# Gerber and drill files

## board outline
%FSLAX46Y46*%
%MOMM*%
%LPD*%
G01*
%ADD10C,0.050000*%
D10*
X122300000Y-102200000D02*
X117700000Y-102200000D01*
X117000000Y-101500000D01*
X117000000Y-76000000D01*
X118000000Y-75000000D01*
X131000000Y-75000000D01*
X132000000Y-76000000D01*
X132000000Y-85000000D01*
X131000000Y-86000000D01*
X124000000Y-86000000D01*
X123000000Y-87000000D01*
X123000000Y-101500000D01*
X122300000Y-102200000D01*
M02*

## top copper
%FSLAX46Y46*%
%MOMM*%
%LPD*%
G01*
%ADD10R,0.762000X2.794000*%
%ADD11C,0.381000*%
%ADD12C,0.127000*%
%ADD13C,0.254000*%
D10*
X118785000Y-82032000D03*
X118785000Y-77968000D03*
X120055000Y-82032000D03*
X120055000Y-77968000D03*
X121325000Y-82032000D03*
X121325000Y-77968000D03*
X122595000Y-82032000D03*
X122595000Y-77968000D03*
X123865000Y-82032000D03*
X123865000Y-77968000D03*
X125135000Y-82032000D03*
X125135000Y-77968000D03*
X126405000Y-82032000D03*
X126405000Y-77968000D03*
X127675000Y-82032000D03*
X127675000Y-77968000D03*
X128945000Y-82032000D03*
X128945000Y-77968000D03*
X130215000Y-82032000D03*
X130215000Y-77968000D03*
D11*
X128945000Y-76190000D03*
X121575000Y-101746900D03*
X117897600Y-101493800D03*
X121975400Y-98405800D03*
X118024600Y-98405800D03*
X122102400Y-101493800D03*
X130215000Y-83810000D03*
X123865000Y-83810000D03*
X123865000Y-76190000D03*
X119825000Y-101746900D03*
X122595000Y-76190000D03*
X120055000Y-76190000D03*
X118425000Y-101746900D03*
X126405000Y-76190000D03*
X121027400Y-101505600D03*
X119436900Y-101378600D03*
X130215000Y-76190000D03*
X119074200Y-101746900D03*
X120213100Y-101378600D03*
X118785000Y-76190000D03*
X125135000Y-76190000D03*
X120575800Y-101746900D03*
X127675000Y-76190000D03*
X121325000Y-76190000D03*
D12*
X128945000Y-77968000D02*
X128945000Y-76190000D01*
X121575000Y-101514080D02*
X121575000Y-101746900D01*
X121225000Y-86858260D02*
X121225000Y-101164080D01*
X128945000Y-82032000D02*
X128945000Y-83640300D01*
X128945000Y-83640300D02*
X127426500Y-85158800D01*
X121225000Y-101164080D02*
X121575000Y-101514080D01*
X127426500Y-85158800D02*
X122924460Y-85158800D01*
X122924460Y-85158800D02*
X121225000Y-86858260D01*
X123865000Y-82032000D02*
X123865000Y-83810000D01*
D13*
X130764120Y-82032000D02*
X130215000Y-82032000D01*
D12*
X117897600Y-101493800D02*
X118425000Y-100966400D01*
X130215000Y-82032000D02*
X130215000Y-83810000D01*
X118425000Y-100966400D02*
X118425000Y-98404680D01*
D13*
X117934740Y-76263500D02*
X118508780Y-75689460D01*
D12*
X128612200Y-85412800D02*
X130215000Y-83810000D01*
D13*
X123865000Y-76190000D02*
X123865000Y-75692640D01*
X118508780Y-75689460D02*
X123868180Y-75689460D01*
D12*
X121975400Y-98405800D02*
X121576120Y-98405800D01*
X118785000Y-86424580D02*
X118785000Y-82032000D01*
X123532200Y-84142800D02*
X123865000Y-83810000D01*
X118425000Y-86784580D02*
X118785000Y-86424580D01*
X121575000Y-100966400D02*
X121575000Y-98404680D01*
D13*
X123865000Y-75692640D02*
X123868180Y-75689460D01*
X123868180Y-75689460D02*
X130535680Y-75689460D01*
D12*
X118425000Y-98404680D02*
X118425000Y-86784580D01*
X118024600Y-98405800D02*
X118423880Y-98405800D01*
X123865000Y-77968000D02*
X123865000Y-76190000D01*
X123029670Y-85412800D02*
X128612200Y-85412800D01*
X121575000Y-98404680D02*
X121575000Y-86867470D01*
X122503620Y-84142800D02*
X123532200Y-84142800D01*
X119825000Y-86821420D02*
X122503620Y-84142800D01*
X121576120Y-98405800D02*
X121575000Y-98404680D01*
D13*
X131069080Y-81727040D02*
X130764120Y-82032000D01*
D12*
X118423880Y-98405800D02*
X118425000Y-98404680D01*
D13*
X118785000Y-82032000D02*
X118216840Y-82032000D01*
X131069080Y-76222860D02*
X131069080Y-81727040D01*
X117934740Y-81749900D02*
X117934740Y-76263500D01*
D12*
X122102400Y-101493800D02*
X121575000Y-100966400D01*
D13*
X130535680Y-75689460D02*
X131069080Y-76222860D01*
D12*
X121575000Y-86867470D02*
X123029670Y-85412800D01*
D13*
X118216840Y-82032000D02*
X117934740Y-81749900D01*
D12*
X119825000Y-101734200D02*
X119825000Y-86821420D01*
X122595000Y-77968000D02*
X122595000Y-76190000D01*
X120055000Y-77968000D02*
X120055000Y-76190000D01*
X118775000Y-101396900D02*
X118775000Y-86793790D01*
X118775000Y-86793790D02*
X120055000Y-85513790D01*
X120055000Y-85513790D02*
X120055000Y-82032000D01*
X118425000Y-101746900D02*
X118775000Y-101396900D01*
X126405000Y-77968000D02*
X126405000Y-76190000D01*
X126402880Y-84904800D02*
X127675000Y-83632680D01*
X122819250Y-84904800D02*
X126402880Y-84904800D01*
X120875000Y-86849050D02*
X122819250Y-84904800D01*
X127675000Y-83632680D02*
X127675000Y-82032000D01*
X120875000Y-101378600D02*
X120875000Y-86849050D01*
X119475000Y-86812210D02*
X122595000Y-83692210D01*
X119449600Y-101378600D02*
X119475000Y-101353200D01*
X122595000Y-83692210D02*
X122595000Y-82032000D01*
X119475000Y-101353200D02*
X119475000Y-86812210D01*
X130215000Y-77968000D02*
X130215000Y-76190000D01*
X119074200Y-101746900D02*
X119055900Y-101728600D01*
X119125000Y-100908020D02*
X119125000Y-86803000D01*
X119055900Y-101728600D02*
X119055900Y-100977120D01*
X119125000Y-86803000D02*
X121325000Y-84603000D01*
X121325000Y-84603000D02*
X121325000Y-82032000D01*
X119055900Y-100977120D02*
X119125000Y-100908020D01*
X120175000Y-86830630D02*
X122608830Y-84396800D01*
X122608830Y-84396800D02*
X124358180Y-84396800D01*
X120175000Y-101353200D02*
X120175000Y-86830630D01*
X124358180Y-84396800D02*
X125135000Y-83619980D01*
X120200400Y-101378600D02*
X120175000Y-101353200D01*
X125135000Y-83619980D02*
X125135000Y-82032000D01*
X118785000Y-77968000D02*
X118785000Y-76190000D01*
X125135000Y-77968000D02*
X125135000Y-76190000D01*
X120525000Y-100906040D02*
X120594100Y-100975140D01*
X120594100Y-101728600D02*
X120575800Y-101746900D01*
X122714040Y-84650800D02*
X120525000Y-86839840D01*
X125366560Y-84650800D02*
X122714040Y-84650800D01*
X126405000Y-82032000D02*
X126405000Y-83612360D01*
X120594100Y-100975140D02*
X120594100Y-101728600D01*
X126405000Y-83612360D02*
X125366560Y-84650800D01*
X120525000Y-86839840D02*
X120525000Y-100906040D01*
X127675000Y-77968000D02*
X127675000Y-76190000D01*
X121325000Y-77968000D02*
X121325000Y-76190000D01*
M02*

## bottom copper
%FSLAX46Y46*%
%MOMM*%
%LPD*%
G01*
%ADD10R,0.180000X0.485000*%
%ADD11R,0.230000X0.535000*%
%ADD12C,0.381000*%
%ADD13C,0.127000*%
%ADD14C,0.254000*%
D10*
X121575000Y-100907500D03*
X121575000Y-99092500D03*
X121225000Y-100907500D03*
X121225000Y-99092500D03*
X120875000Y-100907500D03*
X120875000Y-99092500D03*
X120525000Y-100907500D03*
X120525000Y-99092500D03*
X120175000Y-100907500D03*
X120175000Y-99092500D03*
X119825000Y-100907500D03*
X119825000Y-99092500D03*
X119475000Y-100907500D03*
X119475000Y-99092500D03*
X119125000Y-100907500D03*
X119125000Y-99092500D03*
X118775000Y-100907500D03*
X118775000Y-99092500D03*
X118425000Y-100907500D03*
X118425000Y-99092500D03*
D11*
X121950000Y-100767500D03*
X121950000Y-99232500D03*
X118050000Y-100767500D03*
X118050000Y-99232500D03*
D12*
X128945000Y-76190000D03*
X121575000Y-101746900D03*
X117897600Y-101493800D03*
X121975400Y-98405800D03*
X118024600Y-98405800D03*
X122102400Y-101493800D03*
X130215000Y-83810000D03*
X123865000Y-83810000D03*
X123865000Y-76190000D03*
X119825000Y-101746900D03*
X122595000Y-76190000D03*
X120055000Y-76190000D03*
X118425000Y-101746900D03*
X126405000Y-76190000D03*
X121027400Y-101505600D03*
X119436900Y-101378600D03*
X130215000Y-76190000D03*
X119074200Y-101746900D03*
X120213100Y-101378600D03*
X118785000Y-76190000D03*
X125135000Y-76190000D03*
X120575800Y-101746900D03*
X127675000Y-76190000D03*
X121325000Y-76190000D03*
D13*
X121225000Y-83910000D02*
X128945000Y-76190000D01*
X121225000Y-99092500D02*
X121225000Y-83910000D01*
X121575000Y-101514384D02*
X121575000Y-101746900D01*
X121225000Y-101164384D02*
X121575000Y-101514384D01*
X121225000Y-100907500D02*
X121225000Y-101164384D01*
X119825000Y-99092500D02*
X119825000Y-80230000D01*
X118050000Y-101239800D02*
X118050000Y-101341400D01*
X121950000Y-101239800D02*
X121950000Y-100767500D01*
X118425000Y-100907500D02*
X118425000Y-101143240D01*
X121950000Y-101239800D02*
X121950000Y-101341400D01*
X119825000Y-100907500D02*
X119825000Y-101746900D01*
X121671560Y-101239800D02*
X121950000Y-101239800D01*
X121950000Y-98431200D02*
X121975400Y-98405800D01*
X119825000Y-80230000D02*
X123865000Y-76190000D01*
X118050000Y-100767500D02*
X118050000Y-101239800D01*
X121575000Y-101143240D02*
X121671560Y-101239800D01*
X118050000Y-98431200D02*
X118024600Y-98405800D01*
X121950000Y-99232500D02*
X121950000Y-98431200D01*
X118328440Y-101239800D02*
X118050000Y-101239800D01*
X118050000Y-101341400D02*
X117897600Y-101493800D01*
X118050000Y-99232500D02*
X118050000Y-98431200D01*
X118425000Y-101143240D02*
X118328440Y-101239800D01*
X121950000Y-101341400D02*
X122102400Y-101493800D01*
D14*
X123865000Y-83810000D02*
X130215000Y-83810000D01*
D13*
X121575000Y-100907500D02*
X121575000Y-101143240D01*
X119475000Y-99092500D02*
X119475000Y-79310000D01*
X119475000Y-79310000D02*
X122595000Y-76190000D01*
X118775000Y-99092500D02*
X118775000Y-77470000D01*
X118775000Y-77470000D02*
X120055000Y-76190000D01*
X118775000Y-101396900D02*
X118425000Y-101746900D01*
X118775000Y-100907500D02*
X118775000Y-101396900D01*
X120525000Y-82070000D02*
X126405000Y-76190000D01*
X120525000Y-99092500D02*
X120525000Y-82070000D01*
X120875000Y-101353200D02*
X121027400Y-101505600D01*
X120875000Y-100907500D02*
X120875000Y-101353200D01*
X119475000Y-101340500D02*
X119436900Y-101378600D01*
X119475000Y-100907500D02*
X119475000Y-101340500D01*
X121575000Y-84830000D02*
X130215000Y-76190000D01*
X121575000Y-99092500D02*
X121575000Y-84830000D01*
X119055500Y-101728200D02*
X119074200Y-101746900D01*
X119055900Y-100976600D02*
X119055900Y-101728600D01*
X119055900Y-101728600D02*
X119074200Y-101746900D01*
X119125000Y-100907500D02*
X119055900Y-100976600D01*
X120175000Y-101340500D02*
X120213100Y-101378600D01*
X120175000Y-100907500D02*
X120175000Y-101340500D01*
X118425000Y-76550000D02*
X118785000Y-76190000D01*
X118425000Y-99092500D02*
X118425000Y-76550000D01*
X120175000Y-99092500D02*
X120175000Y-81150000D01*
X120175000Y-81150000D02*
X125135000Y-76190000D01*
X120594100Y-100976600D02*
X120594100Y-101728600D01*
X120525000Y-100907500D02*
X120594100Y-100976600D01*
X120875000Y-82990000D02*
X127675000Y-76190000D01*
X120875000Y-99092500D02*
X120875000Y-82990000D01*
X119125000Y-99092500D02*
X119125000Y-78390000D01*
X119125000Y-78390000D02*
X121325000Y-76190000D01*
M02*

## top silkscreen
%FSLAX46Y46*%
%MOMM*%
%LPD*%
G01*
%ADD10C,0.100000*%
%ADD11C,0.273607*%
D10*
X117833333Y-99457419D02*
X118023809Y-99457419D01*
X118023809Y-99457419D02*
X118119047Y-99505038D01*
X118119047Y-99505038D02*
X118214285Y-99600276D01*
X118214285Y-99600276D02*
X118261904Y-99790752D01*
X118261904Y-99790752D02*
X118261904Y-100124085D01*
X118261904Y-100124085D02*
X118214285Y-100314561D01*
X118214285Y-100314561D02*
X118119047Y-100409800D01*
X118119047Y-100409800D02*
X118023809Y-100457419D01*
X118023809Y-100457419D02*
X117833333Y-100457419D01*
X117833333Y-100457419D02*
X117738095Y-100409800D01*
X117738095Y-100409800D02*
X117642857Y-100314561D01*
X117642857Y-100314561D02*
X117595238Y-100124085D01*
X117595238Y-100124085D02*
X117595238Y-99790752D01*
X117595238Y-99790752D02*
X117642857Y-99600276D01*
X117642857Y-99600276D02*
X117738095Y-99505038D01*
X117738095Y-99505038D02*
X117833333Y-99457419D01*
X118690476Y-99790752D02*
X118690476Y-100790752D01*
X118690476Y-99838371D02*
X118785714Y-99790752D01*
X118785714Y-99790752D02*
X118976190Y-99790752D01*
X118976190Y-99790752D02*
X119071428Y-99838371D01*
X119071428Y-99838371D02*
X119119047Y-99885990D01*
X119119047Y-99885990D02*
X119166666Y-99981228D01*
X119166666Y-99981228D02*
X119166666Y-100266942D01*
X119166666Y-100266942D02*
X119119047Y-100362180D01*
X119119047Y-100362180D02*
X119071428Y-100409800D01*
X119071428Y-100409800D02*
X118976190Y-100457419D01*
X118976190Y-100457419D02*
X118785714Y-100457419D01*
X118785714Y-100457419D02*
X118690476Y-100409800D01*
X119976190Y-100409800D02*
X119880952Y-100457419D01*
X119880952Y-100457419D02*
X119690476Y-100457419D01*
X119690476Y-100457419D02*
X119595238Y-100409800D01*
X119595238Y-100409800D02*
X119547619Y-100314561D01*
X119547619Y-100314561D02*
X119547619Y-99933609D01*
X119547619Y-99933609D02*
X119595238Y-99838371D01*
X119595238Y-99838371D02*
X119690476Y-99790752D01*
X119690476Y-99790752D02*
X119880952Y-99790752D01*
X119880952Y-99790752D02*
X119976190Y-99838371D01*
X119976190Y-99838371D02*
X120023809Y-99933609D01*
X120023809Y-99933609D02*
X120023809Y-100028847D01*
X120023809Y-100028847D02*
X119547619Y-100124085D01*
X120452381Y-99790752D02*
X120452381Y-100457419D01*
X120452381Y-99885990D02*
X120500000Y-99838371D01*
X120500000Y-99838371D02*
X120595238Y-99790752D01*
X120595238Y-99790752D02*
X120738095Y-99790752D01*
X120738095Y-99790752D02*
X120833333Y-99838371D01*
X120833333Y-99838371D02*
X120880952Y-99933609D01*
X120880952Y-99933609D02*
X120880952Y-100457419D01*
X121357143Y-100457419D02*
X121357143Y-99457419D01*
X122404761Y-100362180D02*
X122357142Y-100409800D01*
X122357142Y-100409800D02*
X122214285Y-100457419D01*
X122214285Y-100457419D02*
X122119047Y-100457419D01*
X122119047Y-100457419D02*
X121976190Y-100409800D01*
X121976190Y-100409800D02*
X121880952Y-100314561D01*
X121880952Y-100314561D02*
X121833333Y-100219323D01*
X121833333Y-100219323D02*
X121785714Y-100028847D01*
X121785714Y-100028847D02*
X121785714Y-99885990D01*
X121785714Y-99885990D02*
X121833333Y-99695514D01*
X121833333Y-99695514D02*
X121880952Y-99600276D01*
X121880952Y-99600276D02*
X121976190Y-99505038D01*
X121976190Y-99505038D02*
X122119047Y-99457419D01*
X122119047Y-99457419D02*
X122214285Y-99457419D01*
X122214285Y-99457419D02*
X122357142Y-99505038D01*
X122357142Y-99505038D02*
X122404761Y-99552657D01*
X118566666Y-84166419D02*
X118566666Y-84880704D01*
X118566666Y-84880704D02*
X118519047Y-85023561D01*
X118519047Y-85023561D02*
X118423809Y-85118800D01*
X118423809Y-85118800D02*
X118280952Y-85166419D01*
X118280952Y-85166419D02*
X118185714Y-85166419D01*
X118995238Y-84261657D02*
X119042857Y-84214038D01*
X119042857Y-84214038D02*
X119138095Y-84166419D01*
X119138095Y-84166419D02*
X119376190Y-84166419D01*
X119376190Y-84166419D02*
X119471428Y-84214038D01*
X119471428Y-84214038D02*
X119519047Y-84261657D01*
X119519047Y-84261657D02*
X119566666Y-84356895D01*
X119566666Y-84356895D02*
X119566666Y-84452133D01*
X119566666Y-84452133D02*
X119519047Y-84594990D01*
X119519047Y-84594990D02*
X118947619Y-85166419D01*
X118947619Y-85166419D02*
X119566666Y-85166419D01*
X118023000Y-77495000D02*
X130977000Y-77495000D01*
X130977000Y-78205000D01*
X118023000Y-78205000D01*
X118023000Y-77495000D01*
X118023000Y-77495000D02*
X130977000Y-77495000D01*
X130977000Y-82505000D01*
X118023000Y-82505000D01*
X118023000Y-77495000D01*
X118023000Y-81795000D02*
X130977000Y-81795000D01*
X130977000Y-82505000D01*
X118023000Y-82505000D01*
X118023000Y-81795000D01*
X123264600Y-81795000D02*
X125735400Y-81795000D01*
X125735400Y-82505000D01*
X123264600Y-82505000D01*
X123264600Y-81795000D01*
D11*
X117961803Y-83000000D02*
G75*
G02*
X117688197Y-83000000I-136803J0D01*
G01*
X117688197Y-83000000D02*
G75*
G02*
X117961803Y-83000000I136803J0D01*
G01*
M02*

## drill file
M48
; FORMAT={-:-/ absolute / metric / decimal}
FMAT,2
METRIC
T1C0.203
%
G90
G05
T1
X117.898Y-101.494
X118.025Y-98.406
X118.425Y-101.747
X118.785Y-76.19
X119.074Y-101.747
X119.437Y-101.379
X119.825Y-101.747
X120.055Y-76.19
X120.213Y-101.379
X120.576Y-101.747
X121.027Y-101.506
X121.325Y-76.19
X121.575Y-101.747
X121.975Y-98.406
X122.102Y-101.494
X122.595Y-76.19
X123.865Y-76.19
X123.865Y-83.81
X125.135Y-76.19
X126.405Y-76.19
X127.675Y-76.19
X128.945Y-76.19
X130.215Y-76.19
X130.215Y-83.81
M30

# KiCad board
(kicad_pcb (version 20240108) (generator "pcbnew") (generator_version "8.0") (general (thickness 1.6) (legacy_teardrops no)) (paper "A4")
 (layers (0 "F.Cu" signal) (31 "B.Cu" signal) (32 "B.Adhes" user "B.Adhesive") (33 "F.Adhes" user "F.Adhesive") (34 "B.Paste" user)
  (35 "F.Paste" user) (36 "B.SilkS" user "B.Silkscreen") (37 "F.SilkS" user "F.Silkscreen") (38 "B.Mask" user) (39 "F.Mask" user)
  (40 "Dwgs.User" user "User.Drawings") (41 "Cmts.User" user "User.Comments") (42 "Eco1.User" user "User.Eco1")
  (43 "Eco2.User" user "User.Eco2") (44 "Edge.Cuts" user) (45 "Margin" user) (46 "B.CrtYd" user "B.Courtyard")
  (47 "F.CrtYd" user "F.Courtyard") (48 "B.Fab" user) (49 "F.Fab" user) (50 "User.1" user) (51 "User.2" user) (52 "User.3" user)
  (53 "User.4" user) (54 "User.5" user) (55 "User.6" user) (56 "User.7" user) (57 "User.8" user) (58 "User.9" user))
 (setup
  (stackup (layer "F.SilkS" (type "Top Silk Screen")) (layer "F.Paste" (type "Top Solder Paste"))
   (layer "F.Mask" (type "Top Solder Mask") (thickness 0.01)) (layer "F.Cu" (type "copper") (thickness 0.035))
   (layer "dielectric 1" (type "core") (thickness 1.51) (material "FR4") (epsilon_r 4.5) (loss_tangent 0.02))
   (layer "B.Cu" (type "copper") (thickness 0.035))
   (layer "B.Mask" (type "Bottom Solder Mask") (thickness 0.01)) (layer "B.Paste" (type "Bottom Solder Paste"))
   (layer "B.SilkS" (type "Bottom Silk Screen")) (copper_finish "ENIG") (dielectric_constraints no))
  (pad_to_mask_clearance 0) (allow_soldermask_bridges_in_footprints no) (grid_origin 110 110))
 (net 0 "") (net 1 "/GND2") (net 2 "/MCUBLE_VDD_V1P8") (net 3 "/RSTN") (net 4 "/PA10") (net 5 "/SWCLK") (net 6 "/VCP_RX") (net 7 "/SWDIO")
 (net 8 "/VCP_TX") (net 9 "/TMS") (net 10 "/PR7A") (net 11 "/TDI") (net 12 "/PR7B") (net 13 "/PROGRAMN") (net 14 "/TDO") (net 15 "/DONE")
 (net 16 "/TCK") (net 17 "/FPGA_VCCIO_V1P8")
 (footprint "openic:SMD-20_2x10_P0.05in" (layer "F.Cu") (at 124.5 80)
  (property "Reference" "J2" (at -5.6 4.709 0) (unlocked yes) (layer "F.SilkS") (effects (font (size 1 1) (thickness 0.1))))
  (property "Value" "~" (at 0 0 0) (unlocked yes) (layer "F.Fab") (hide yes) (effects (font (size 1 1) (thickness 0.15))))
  (fp_rect (start -6.477 -2.505) (end 6.477 -1.795) (stroke (width 0.1) (type default)) (fill none) (layer "F.SilkS"))
  (fp_rect (start -6.477 -2.505) (end 6.477 2.505) (stroke (width 0.1) (type default)) (fill none) (layer "F.SilkS"))
  (fp_rect (start -6.477 1.795) (end 6.477 2.505) (stroke (width 0.1) (type default)) (fill none) (layer "F.SilkS"))
  (fp_rect (start -1.2354 1.795) (end 1.2354 2.505) (stroke (width 0.1) (type default)) (fill none) (layer "F.SilkS"))
  (fp_circle (center -6.675 3) (end -6.475 2.9) (stroke (width 0.1) (type default)) (fill solid) (layer "F.SilkS"))
  (pad "1" smd rect (at -5.715 2.032) (size 0.762 2.794) (layers "F.Cu" "F.Paste" "F.Mask") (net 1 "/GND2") (thermal_bridge_angle 45))
  (pad "2" smd rect (at -5.715 -2.032) (size 0.762 2.794) (layers "F.Cu" "F.Paste" "F.Mask") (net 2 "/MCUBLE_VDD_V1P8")
   (thermal_bridge_angle 45))
  (pad "3" smd rect (at -4.445 2.032) (size 0.762 2.794) (layers "F.Cu" "F.Paste" "F.Mask") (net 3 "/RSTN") (thermal_bridge_angle 45))
  (pad "4" smd rect (at -4.445 -2.032) (size 0.762 2.794) (layers "F.Cu" "F.Paste" "F.Mask") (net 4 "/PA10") (thermal_bridge_angle 45))
  (pad "5" smd rect (at -3.175 2.032) (size 0.762 2.794) (layers "F.Cu" "F.Paste" "F.Mask") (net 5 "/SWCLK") (thermal_bridge_angle 45))
  (pad "6" smd rect (at -3.175 -2.032) (size 0.762 2.794) (layers "F.Cu" "F.Paste" "F.Mask") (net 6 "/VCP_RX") (thermal_bridge_angle 45))
  (pad "7" smd rect (at -1.905 2.032) (size 0.762 2.794) (layers "F.Cu" "F.Paste" "F.Mask") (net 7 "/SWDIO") (thermal_bridge_angle 45))
  (pad "8" smd rect (at -1.905 -2.032) (size 0.762 2.794) (layers "F.Cu" "F.Paste" "F.Mask") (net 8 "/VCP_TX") (thermal_bridge_angle 45))
  (pad "9" smd rect (at -0.635 2.032) (size 0.762 2.794) (layers "F.Cu" "F.Paste" "F.Mask") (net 1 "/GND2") (thermal_bridge_angle 45))
  (pad "10" smd rect (at -0.635 -2.032) (size 0.762 2.794) (layers "F.Cu" "F.Paste" "F.Mask") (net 1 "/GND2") (thermal_bridge_angle 45))
  (pad "11" smd rect (at 0.635 2.032) (size 0.762 2.794) (layers "F.Cu" "F.Paste" "F.Mask") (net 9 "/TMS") (thermal_bridge_angle 45))
  (pad "12" smd rect (at 0.635 -2.032) (size 0.762 2.794) (layers "F.Cu" "F.Paste" "F.Mask") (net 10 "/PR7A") (thermal_bridge_angle 45))
  (pad "13" smd rect (at 1.905 2.032) (size 0.762 2.794) (layers "F.Cu" "F.Paste" "F.Mask") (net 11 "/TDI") (thermal_bridge_angle 45))
  (pad "14" smd rect (at 1.905 -2.032) (size 0.762 2.794) (layers "F.Cu" "F.Paste" "F.Mask") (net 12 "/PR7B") (thermal_bridge_angle 45))
  (pad "15" smd rect (at 3.175 2.032) (size 0.762 2.794) (layers "F.Cu" "F.Paste" "F.Mask") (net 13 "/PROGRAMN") (thermal_bridge_angle 45))
  (pad "16" smd rect (at 3.175 -2.032) (size 0.762 2.794) (layers "F.Cu" "F.Paste" "F.Mask") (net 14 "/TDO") (thermal_bridge_angle 45))
  (pad "17" smd rect (at 4.445 2.032) (size 0.762 2.794) (layers "F.Cu" "F.Paste" "F.Mask") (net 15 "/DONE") (thermal_bridge_angle 45))
  (pad "18" smd rect (at 4.445 -2.032) (size 0.762 2.794) (layers "F.Cu" "F.Paste" "F.Mask") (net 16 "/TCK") (thermal_bridge_angle 45))
  (pad "19" smd rect (at 5.715 2.032) (size 0.762 2.794) (layers "F.Cu" "F.Paste" "F.Mask") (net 1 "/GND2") (thermal_bridge_angle 45))
  (pad "20" smd rect (at 5.715 -2.032) (size 0.762 2.794) (layers "F.Cu" "F.Paste" "F.Mask") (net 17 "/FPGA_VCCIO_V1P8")
   (thermal_bridge_angle 45)))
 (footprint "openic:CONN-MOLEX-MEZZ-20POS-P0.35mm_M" (layer "B.Cu") (at 120 100 180)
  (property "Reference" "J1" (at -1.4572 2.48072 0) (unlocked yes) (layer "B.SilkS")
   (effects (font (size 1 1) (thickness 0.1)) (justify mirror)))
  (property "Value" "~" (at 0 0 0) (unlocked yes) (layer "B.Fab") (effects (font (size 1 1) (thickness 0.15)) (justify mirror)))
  (pad "1" smd rect (at -1.575 -0.9075 180) (size 0.18 0.485) (layers "B.Cu" "B.Paste" "B.Mask") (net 1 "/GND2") (thermal_bridge_angle 45))
  (pad "2" smd rect (at -1.575 0.9075 180) (size 0.18 0.485) (layers "B.Cu" "B.Paste" "B.Mask") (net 17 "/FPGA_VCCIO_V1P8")
   (thermal_bridge_angle 45))
  (pad "3" smd rect (at -1.225 -0.9075 180) (size 0.18 0.485) (layers "B.Cu" "B.Paste" "B.Mask") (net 15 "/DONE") (thermal_bridge_angle 45))
  (pad "4" smd rect (at -1.225 0.9075 180) (size 0.18 0.485) (layers "B.Cu" "B.Paste" "B.Mask") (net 16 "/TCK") (thermal_bridge_angle 45))
  (pad "5" smd rect (at -0.875 -0.9075 180) (size 0.18 0.485) (layers "B.Cu" "B.Paste" "B.Mask") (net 13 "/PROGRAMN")
   (thermal_bridge_angle 45))
  (pad "6" smd rect (at -0.875 0.9075 180) (size 0.18 0.485) (layers "B.Cu" "B.Paste" "B.Mask") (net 14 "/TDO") (thermal_bridge_angle 45))
  (pad "7" smd rect (at -0.525 -0.9075 180) (size 0.18 0.485) (layers "B.Cu" "B.Paste" "B.Mask") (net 11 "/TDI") (thermal_bridge_angle 45))
  (pad "8" smd rect (at -0.525 0.9075 180) (size 0.18 0.485) (layers "B.Cu" "B.Paste" "B.Mask") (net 12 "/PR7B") (thermal_bridge_angle 45))
  (pad "9" smd rect (at -0.175 -0.9075 180) (size 0.18 0.485) (layers "B.Cu" "B.Paste" "B.Mask") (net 9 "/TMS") (thermal_bridge_angle 45))
  (pad "10" smd rect (at -0.175 0.9075 180) (size 0.18 0.485) (layers "B.Cu" "B.Paste" "B.Mask") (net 10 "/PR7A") (thermal_bridge_angle 45))
  (pad "11" smd rect (at 0.175 -0.9075 180) (size 0.18 0.485) (layers "B.Cu" "B.Paste" "B.Mask") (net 1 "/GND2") (thermal_bridge_angle 45))
  (pad "12" smd rect (at 0.175 0.9075 180) (size 0.18 0.485) (layers "B.Cu" "B.Paste" "B.Mask") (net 1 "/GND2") (thermal_bridge_angle 45))
  (pad "13" smd rect (at 0.525 -0.9075 180) (size 0.18 0.485) (layers "B.Cu" "B.Paste" "B.Mask") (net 7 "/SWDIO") (thermal_bridge_angle 45))
  (pad "14" smd rect (at 0.525 0.9075 180) (size 0.18 0.485) (layers "B.Cu" "B.Paste" "B.Mask") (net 8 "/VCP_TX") (thermal_bridge_angle 45))
  (pad "15" smd rect (at 0.875 -0.9075 180) (size 0.18 0.485) (layers "B.Cu" "B.Paste" "B.Mask") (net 5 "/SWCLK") (thermal_bridge_angle 45))
  (pad "16" smd rect (at 0.875 0.9075 180) (size 0.18 0.485) (layers "B.Cu" "B.Paste" "B.Mask") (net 6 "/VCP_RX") (thermal_bridge_angle 45))
  (pad "17" smd rect (at 1.225 -0.9075 180) (size 0.18 0.485) (layers "B.Cu" "B.Paste" "B.Mask") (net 3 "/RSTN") (thermal_bridge_angle 45))
  (pad "18" smd rect (at 1.225 0.9075 180) (size 0.18 0.485) (layers "B.Cu" "B.Paste" "B.Mask") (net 4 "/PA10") (thermal_bridge_angle 45))
  (pad "19" smd rect (at 1.575 -0.9075 180) (size 0.18 0.485) (layers "B.Cu" "B.Paste" "B.Mask") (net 1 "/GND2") (thermal_bridge_angle 45))
  (pad "20" smd rect (at 1.575 0.9075 180) (size 0.18 0.485) (layers "B.Cu" "B.Paste" "B.Mask") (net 2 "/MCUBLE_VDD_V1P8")
   (thermal_bridge_angle 45))
  (pad "P1" smd rect (at -1.95 -0.7675 180) (size 0.23 0.535) (layers "B.Cu" "B.Paste" "B.Mask") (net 1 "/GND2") (thermal_bridge_angle 45))
  (pad "P2" smd rect (at -1.95 0.7675 180) (size 0.23 0.535) (layers "B.Cu" "B.Paste" "B.Mask") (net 1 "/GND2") (thermal_bridge_angle 45))
  (pad "P3" smd rect (at 1.95 -0.7675 180) (size 0.23 0.535) (layers "B.Cu" "B.Paste" "B.Mask") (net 1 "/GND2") (thermal_bridge_angle 45))
  (pad "P4" smd rect (at 1.95 0.7675 180) (size 0.23 0.535) (layers "B.Cu" "B.Paste" "B.Mask") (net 1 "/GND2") (thermal_bridge_angle 45))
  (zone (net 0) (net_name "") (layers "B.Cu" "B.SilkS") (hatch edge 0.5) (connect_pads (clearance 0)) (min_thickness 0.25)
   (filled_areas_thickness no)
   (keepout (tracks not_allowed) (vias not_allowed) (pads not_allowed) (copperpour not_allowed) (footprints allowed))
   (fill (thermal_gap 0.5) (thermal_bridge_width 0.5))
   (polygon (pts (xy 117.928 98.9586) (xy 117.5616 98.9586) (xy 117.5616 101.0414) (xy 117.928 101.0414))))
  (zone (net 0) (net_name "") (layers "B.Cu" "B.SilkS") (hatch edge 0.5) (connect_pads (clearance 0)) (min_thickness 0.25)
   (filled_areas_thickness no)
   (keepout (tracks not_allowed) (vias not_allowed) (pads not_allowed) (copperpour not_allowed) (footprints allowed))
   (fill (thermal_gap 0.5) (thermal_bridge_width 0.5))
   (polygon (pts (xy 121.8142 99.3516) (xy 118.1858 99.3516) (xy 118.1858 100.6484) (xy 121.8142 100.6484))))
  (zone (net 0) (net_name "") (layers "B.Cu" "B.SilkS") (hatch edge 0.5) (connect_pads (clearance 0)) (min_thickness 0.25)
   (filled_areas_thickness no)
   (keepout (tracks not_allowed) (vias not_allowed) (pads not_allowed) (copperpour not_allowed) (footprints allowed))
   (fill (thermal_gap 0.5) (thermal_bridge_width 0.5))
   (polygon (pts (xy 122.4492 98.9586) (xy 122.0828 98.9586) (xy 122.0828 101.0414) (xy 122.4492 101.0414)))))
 (gr_poly
  (pts (xy 122.3 102.2) (xy 117.7 102.2) (xy 117 101.5) (xy 117 76) (xy 118 75) (xy 131 75) (xy 132 76) (xy 132 85) (xy 131 86) (xy 124 86)
   (xy 123 87) (xy 123 101.5))
  (stroke (width 0.05) (type solid)) (fill none) (layer "Edge.Cuts"))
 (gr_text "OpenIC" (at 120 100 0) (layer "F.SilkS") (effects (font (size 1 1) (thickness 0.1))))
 (segment (start 128.945 77.968) (end 128.945 76.19) (width 0.127) (layer "F.Cu") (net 16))
 (via (at 128.945 76.19) (size 0.381) (drill 0.2032) (layers "F.Cu" "B.Cu") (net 16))
 (segment (start 121.225 83.91) (end 128.945 76.19) (width 0.127) (layer "B.Cu") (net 16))
 (segment (start 121.225 99.0925) (end 121.225 83.91) (width 0.127) (layer "B.Cu") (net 16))
 (segment (start 121.575 101.51408) (end 121.575 101.7469) (width 0.127) (layer "F.Cu") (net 15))
 (segment (start 121.225 86.85826) (end 121.225 101.16408) (width 0.127) (layer "F.Cu") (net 15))
 (segment (start 128.945 82.032) (end 128.945 83.6403) (width 0.127) (layer "F.Cu") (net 15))
 (segment (start 128.945 83.6403) (end 127.4265 85.1588) (width 0.127) (layer "F.Cu") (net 15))
 (segment (start 121.225 101.16408) (end 121.575 101.51408) (width 0.127) (layer "F.Cu") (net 15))
 (segment (start 127.4265 85.1588) (end 122.92446 85.1588) (width 0.127) (layer "F.Cu") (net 15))
 (segment (start 122.92446 85.1588) (end 121.225 86.85826) (width 0.127) (layer "F.Cu") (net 15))
 (via (at 121.575 101.7469) (size 0.381) (drill 0.2032) (layers "F.Cu" "B.Cu") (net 15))
 (segment (start 121.575 101.514384) (end 121.575 101.7469) (width 0.127) (layer "B.Cu") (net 15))
 (segment (start 121.225 101.164384) (end 121.575 101.514384) (width 0.127) (layer "B.Cu") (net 15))
 (segment (start 121.225 100.9075) (end 121.225 101.164384) (width 0.127) (layer "B.Cu") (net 15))
 (segment (start 123.865 82.032) (end 123.865 83.81) (width 0.127) (layer "F.Cu") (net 1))
 (segment (start 130.76412 82.032) (end 130.215 82.032) (width 0.254) (layer "F.Cu") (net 1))
 (segment (start 117.8976 101.4938) (end 118.425 100.9664) (width 0.127) (layer "F.Cu") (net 1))
 (segment (start 130.215 82.032) (end 130.215 83.81) (width 0.127) (layer "F.Cu") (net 1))
 (segment (start 118.425 100.9664) (end 118.425 98.40468) (width 0.127) (layer "F.Cu") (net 1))
 (segment (start 117.93474 76.2635) (end 118.50878 75.68946) (width 0.254) (layer "F.Cu") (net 1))
 (segment (start 128.6122 85.4128) (end 130.215 83.81) (width 0.127) (layer "F.Cu") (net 1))
 (segment (start 123.865 76.19) (end 123.865 75.69264) (width 0.254) (layer "F.Cu") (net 1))
 (segment (start 118.50878 75.68946) (end 123.86818 75.68946) (width 0.254) (layer "F.Cu") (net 1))
 (segment (start 121.9754 98.4058) (end 121.57612 98.4058) (width 0.127) (layer "F.Cu") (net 1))
 (segment (start 118.785 86.42458) (end 118.785 82.032) (width 0.127) (layer "F.Cu") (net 1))
 (segment (start 123.5322 84.1428) (end 123.865 83.81) (width 0.127) (layer "F.Cu") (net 1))
 (segment (start 118.425 86.78458) (end 118.785 86.42458) (width 0.127) (layer "F.Cu") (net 1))
 (segment (start 121.575 100.9664) (end 121.575 98.40468) (width 0.127) (layer "F.Cu") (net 1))
 (segment (start 123.865 75.69264) (end 123.86818 75.68946) (width 0.254) (layer "F.Cu") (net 1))
 (segment (start 123.86818 75.68946) (end 130.53568 75.68946) (width 0.254) (layer "F.Cu") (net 1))
 (segment (start 118.425 98.40468) (end 118.425 86.78458) (width 0.127) (layer "F.Cu") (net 1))
 (segment (start 118.0246 98.4058) (end 118.42388 98.4058) (width 0.127) (layer "F.Cu") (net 1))
 (segment (start 123.865 77.968) (end 123.865 76.19) (width 0.127) (layer "F.Cu") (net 1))
 (segment (start 123.02967 85.4128) (end 128.6122 85.4128) (width 0.127) (layer "F.Cu") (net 1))
 (segment (start 121.575 98.40468) (end 121.575 86.86747) (width 0.127) (layer "F.Cu") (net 1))
 (segment (start 122.50362 84.1428) (end 123.5322 84.1428) (width 0.127) (layer "F.Cu") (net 1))
 (segment (start 119.825 86.82142) (end 122.50362 84.1428) (width 0.127) (layer "F.Cu") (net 1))
 (segment (start 121.57612 98.4058) (end 121.575 98.40468) (width 0.127) (layer "F.Cu") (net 1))
 (segment (start 131.06908 81.72704) (end 130.76412 82.032) (width 0.254) (layer "F.Cu") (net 1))
 (segment (start 118.42388 98.4058) (end 118.425 98.40468) (width 0.127) (layer "F.Cu") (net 1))
 (segment (start 118.785 82.032) (end 118.21684 82.032) (width 0.254) (layer "F.Cu") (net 1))
 (segment (start 131.06908 76.22286) (end 131.06908 81.72704) (width 0.254) (layer "F.Cu") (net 1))
 (segment (start 117.93474 81.7499) (end 117.93474 76.2635) (width 0.254) (layer "F.Cu") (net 1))
 (segment (start 122.1024 101.4938) (end 121.575 100.9664) (width 0.127) (layer "F.Cu") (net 1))
 (segment (start 130.53568 75.68946) (end 131.06908 76.22286) (width 0.254) (layer "F.Cu") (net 1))
 (segment (start 121.575 86.86747) (end 123.02967 85.4128) (width 0.127) (layer "F.Cu") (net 1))
 (segment (start 118.21684 82.032) (end 117.93474 81.7499) (width 0.254) (layer "F.Cu") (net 1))
 (segment (start 119.825 101.7342) (end 119.825 86.82142) (width 0.127) (layer "F.Cu") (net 1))
 (via (at 117.8976 101.4938) (size 0.381) (drill 0.2032) (layers "F.Cu" "B.Cu") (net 1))
 (via (at 121.9754 98.4058) (size 0.381) (drill 0.2032) (layers "F.Cu" "B.Cu") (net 1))
 (via (at 118.0246 98.4058) (size 0.381) (drill 0.2032) (layers "F.Cu" "B.Cu") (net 1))
 (via (at 122.1024 101.4938) (size 0.381) (drill 0.2032) (layers "F.Cu" "B.Cu") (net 1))
 (via (at 130.215 83.81) (size 0.381) (drill 0.2032) (layers "F.Cu" "B.Cu") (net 1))
 (via (at 123.865 83.81) (size 0.381) (drill 0.2032) (layers "F.Cu" "B.Cu") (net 1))
 (via (at 123.865 76.19) (size 0.381) (drill 0.2032) (layers "F.Cu" "B.Cu") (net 1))
 (via (at 119.825 101.7469) (size 0.381) (drill 0.2032) (layers "F.Cu" "B.Cu") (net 1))
 (segment (start 119.825 99.0925) (end 119.825 80.23) (width 0.127) (layer "B.Cu") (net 1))
 (segment (start 118.05 101.2398) (end 118.05 101.3414) (width 0.127) (layer "B.Cu") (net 1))
 (segment (start 121.95 101.2398) (end 121.95 100.7675) (width 0.127) (layer "B.Cu") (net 1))
 (segment (start 118.425 100.9075) (end 118.425 101.14324) (width 0.127) (layer "B.Cu") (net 1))
 (segment (start 121.95 101.2398) (end 121.95 101.3414) (width 0.127) (layer "B.Cu") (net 1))
 (segment (start 119.825 100.9075) (end 119.825 101.7469) (width 0.127) (layer "B.Cu") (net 1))
 (segment (start 121.67156 101.2398) (end 121.95 101.2398) (width 0.127) (layer "B.Cu") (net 1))
 (segment (start 121.95 98.4312) (end 121.9754 98.4058) (width 0.127) (layer "B.Cu") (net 1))
 (segment (start 119.825 80.23) (end 123.865 76.19) (width 0.127) (layer "B.Cu") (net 1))
 (segment (start 118.05 100.7675) (end 118.05 101.2398) (width 0.127) (layer "B.Cu") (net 1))
 (segment (start 121.575 101.14324) (end 121.67156 101.2398) (width 0.127) (layer "B.Cu") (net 1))
 (segment (start 118.05 98.4312) (end 118.0246 98.4058) (width 0.127) (layer "B.Cu") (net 1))
 (segment (start 121.95 99.2325) (end 121.95 98.4312) (width 0.127) (layer "B.Cu") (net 1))
 (segment (start 118.32844 101.2398) (end 118.05 101.2398) (width 0.127) (layer "B.Cu") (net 1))
 (segment (start 118.05 101.3414) (end 117.8976 101.4938) (width 0.127) (layer "B.Cu") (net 1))
 (segment (start 118.05 99.2325) (end 118.05 98.4312) (width 0.127) (layer "B.Cu") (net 1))
 (segment (start 118.425 101.14324) (end 118.32844 101.2398) (width 0.127) (layer "B.Cu") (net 1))
 (segment (start 121.95 101.3414) (end 122.1024 101.4938) (width 0.127) (layer "B.Cu") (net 1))
 (segment (start 123.865 83.81) (end 130.215 83.81) (width 0.254) (layer "B.Cu") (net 1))
 (segment (start 121.575 100.9075) (end 121.575 101.14324) (width 0.127) (layer "B.Cu") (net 1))
 (segment (start 122.595 77.968) (end 122.595 76.19) (width 0.127) (layer "F.Cu") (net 8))
 (via (at 122.595 76.19) (size 0.381) (drill 0.2032) (layers "F.Cu" "B.Cu") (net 8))
 (segment (start 119.475 99.0925) (end 119.475 79.31) (width 0.127) (layer "B.Cu") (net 8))
 (segment (start 119.475 79.31) (end 122.595 76.19) (width 0.127) (layer "B.Cu") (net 8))
 (segment (start 120.055 77.968) (end 120.055 76.19) (width 0.127) (layer "F.Cu") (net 4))
 (via (at 120.055 76.19) (size 0.381) (drill 0.2032) (layers "F.Cu" "B.Cu") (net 4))
 (segment (start 118.775 99.0925) (end 118.775 77.47) (width 0.127) (layer "B.Cu") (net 4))
 (segment (start 118.775 77.47) (end 120.055 76.19) (width 0.127) (layer "B.Cu") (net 4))
 (segment (start 118.775 101.3969) (end 118.775 86.79379) (width 0.127) (layer "F.Cu") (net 3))
 (segment (start 118.775 86.79379) (end 120.055 85.51379) (width 0.127) (layer "F.Cu") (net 3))
 (segment (start 120.055 85.51379) (end 120.055 82.032) (width 0.127) (layer "F.Cu") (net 3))
 (segment (start 118.425 101.7469) (end 118.775 101.3969) (width 0.127) (layer "F.Cu") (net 3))
 (via (at 118.425 101.7469) (size 0.381) (drill 0.2032) (layers "F.Cu" "B.Cu") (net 3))
 (segment (start 118.775 101.3969) (end 118.425 101.7469) (width 0.127) (layer "B.Cu") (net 3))
 (segment (start 118.775 100.9075) (end 118.775 101.3969) (width 0.127) (layer "B.Cu") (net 3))
 (segment (start 126.405 77.968) (end 126.405 76.19) (width 0.127) (layer "F.Cu") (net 12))
 (via (at 126.405 76.19) (size 0.381) (drill 0.2032) (layers "F.Cu" "B.Cu") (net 12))
 (segment (start 120.525 82.07) (end 126.405 76.19) (width 0.127) (layer "B.Cu") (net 12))
 (segment (start 120.525 99.0925) (end 120.525 82.07) (width 0.127) (layer "B.Cu") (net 12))
 (segment (start 126.40288 84.9048) (end 127.675 83.63268) (width 0.127) (layer "F.Cu") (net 13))
 (segment (start 122.81925 84.9048) (end 126.40288 84.9048) (width 0.127) (layer "F.Cu") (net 13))
 (segment (start 120.875 86.84905) (end 122.81925 84.9048) (width 0.127) (layer "F.Cu") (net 13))
 (segment (start 127.675 83.63268) (end 127.675 82.032) (width 0.127) (layer "F.Cu") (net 13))
 (segment (start 120.875 101.3786) (end 120.875 86.84905) (width 0.127) (layer "F.Cu") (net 13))
 (via (at 121.0274 101.5056) (size 0.381) (drill 0.2032) (layers "F.Cu" "B.Cu") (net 13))
 (segment (start 120.875 101.3532) (end 121.0274 101.5056) (width 0.127) (layer "B.Cu") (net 13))
 (segment (start 120.875 100.9075) (end 120.875 101.3532) (width 0.127) (layer "B.Cu") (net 13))
 (segment (start 119.475 86.81221) (end 122.595 83.69221) (width 0.127) (layer "F.Cu") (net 7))
 (segment (start 119.4496 101.3786) (end 119.475 101.3532) (width 0.127) (layer "F.Cu") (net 7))
 (segment (start 122.595 83.69221) (end 122.595 82.032) (width 0.127) (layer "F.Cu") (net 7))
 (segment (start 119.475 101.3532) (end 119.475 86.81221) (width 0.127) (layer "F.Cu") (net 7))
 (via (at 119.4369 101.3786) (size 0.381) (drill 0.2032) (layers "F.Cu" "B.Cu") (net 7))
 (segment (start 119.475 101.3405) (end 119.4369 101.3786) (width 0.127) (layer "B.Cu") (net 7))
 (segment (start 119.475 100.9075) (end 119.475 101.3405) (width 0.127) (layer "B.Cu") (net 7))
 (segment (start 130.215 77.968) (end 130.215 76.19) (width 0.127) (layer "F.Cu") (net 17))
 (via (at 130.215 76.19) (size 0.381) (drill 0.2032) (layers "F.Cu" "B.Cu") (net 17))
 (segment (start 121.575 84.83) (end 130.215 76.19) (width 0.127) (layer "B.Cu") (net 17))
 (segment (start 121.575 99.0925) (end 121.575 84.83) (width 0.127) (layer "B.Cu") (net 17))
 (segment (start 119.0742 101.7469) (end 119.0559 101.7286) (width 0.127) (layer "F.Cu") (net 5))
 (segment (start 119.125 100.90802) (end 119.125 86.803) (width 0.127) (layer "F.Cu") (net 5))
 (segment (start 119.0559 101.7286) (end 119.0559 100.97712) (width 0.127) (layer "F.Cu") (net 5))
 (segment (start 119.125 86.803) (end 121.325 84.603) (width 0.127) (layer "F.Cu") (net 5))
 (segment (start 121.325 84.603) (end 121.325 82.032) (width 0.127) (layer "F.Cu") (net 5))
 (segment (start 119.0559 100.97712) (end 119.125 100.90802) (width 0.127) (layer "F.Cu") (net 5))
 (via (at 119.0742 101.7469) (size 0.381) (drill 0.2032) (layers "F.Cu" "B.Cu") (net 5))
 (segment (start 119.0555 101.7282) (end 119.0742 101.7469) (width 0.127) (layer "B.Cu") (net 5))
 (segment (start 119.0559 100.9766) (end 119.0559 101.7286) (width 0.127) (layer "B.Cu") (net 5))
 (segment (start 119.0559 101.7286) (end 119.0742 101.7469) (width 0.127) (layer "B.Cu") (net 5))
 (segment (start 119.125 100.9075) (end 119.0559 100.9766) (width 0.127) (layer "B.Cu") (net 5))
 (segment (start 120.175 86.83063) (end 122.60883 84.3968) (width 0.127) (layer "F.Cu") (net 9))
 (segment (start 122.60883 84.3968) (end 124.35818 84.3968) (width 0.127) (layer "F.Cu") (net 9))
 (segment (start 120.175 101.3532) (end 120.175 86.83063) (width 0.127) (layer "F.Cu") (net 9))
 (segment (start 124.35818 84.3968) (end 125.135 83.61998) (width 0.127) (layer "F.Cu") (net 9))
 (segment (start 120.2004 101.3786) (end 120.175 101.3532) (width 0.127) (layer "F.Cu") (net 9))
 (segment (start 125.135 83.61998) (end 125.135 82.032) (width 0.127) (layer "F.Cu") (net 9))
 (via (at 120.2131 101.3786) (size 0.381) (drill 0.2032) (layers "F.Cu" "B.Cu") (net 9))
 (segment (start 120.175 101.3405) (end 120.2131 101.3786) (width 0.127) (layer "B.Cu") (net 9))
 (segment (start 120.175 100.9075) (end 120.175 101.3405) (width 0.127) (layer "B.Cu") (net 9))
 (segment (start 118.785 77.968) (end 118.785 76.19) (width 0.127) (layer "F.Cu") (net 2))
 (via (at 118.785 76.19) (size 0.381) (drill 0.2032) (layers "F.Cu" "B.Cu") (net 2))
 (segment (start 118.425 76.55) (end 118.785 76.19) (width 0.127) (layer "B.Cu") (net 2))
 (segment (start 118.425 99.0925) (end 118.425 76.55) (width 0.127) (layer "B.Cu") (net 2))
 (segment (start 125.135 77.968) (end 125.135 76.19) (width 0.127) (layer "F.Cu") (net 10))
 (via (at 125.135 76.19) (size 0.381) (drill 0.2032) (layers "F.Cu" "B.Cu") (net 10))
 (segment (start 120.175 99.0925) (end 120.175 81.15) (width 0.127) (layer "B.Cu") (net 10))
 (segment (start 120.175 81.15) (end 125.135 76.19) (width 0.127) (layer "B.Cu") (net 10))
 (segment (start 120.525 100.90604) (end 120.5941 100.97514) (width 0.127) (layer "F.Cu") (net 11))
 (segment (start 120.5941 101.7286) (end 120.5758 101.7469) (width 0.127) (layer "F.Cu") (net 11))
 (segment (start 122.71404 84.6508) (end 120.525 86.83984) (width 0.127) (layer "F.Cu") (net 11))
 (segment (start 125.36656 84.6508) (end 122.71404 84.6508) (width 0.127) (layer "F.Cu") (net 11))
 (segment (start 126.405 82.032) (end 126.405 83.61236) (width 0.127) (layer "F.Cu") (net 11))
 (segment (start 120.5941 100.97514) (end 120.5941 101.7286) (width 0.127) (layer "F.Cu") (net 11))
 (segment (start 126.405 83.61236) (end 125.36656 84.6508) (width 0.127) (layer "F.Cu") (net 11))
 (segment (start 120.525 86.83984) (end 120.525 100.90604) (width 0.127) (layer "F.Cu") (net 11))
 (via (at 120.5758 101.7469) (size 0.381) (drill 0.2032) (layers "F.Cu" "B.Cu") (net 11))
 (segment (start 120.5941 100.9766) (end 120.5941 101.7286) (width 0.127) (layer "B.Cu") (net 11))
 (segment (start 120.525 100.9075) (end 120.5941 100.9766) (width 0.127) (layer "B.Cu") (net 11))
 (segment (start 127.675 77.968) (end 127.675 76.19) (width 0.127) (layer "F.Cu") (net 14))
 (via (at 127.675 76.19) (size 0.381) (drill 0.2032) (layers "F.Cu" "B.Cu") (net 14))
 (segment (start 120.875 82.99) (end 127.675 76.19) (width 0.127) (layer "B.Cu") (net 14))
 (segment (start 120.875 99.0925) (end 120.875 82.99) (width 0.127) (layer "B.Cu") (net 14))
 (segment (start 121.325 77.968) (end 121.325 76.19) (width 0.127) (layer "F.Cu") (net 6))
 (via (at 121.325 76.19) (size 0.381) (drill 0.2032) (layers "F.Cu" "B.Cu") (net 6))
 (segment (start 119.125 99.0925) (end 119.125 78.39) (width 0.127) (layer "B.Cu") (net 6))
 (segment (start 119.125 78.39) (end 121.325 76.19) (width 0.127) (layer "B.Cu") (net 6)))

